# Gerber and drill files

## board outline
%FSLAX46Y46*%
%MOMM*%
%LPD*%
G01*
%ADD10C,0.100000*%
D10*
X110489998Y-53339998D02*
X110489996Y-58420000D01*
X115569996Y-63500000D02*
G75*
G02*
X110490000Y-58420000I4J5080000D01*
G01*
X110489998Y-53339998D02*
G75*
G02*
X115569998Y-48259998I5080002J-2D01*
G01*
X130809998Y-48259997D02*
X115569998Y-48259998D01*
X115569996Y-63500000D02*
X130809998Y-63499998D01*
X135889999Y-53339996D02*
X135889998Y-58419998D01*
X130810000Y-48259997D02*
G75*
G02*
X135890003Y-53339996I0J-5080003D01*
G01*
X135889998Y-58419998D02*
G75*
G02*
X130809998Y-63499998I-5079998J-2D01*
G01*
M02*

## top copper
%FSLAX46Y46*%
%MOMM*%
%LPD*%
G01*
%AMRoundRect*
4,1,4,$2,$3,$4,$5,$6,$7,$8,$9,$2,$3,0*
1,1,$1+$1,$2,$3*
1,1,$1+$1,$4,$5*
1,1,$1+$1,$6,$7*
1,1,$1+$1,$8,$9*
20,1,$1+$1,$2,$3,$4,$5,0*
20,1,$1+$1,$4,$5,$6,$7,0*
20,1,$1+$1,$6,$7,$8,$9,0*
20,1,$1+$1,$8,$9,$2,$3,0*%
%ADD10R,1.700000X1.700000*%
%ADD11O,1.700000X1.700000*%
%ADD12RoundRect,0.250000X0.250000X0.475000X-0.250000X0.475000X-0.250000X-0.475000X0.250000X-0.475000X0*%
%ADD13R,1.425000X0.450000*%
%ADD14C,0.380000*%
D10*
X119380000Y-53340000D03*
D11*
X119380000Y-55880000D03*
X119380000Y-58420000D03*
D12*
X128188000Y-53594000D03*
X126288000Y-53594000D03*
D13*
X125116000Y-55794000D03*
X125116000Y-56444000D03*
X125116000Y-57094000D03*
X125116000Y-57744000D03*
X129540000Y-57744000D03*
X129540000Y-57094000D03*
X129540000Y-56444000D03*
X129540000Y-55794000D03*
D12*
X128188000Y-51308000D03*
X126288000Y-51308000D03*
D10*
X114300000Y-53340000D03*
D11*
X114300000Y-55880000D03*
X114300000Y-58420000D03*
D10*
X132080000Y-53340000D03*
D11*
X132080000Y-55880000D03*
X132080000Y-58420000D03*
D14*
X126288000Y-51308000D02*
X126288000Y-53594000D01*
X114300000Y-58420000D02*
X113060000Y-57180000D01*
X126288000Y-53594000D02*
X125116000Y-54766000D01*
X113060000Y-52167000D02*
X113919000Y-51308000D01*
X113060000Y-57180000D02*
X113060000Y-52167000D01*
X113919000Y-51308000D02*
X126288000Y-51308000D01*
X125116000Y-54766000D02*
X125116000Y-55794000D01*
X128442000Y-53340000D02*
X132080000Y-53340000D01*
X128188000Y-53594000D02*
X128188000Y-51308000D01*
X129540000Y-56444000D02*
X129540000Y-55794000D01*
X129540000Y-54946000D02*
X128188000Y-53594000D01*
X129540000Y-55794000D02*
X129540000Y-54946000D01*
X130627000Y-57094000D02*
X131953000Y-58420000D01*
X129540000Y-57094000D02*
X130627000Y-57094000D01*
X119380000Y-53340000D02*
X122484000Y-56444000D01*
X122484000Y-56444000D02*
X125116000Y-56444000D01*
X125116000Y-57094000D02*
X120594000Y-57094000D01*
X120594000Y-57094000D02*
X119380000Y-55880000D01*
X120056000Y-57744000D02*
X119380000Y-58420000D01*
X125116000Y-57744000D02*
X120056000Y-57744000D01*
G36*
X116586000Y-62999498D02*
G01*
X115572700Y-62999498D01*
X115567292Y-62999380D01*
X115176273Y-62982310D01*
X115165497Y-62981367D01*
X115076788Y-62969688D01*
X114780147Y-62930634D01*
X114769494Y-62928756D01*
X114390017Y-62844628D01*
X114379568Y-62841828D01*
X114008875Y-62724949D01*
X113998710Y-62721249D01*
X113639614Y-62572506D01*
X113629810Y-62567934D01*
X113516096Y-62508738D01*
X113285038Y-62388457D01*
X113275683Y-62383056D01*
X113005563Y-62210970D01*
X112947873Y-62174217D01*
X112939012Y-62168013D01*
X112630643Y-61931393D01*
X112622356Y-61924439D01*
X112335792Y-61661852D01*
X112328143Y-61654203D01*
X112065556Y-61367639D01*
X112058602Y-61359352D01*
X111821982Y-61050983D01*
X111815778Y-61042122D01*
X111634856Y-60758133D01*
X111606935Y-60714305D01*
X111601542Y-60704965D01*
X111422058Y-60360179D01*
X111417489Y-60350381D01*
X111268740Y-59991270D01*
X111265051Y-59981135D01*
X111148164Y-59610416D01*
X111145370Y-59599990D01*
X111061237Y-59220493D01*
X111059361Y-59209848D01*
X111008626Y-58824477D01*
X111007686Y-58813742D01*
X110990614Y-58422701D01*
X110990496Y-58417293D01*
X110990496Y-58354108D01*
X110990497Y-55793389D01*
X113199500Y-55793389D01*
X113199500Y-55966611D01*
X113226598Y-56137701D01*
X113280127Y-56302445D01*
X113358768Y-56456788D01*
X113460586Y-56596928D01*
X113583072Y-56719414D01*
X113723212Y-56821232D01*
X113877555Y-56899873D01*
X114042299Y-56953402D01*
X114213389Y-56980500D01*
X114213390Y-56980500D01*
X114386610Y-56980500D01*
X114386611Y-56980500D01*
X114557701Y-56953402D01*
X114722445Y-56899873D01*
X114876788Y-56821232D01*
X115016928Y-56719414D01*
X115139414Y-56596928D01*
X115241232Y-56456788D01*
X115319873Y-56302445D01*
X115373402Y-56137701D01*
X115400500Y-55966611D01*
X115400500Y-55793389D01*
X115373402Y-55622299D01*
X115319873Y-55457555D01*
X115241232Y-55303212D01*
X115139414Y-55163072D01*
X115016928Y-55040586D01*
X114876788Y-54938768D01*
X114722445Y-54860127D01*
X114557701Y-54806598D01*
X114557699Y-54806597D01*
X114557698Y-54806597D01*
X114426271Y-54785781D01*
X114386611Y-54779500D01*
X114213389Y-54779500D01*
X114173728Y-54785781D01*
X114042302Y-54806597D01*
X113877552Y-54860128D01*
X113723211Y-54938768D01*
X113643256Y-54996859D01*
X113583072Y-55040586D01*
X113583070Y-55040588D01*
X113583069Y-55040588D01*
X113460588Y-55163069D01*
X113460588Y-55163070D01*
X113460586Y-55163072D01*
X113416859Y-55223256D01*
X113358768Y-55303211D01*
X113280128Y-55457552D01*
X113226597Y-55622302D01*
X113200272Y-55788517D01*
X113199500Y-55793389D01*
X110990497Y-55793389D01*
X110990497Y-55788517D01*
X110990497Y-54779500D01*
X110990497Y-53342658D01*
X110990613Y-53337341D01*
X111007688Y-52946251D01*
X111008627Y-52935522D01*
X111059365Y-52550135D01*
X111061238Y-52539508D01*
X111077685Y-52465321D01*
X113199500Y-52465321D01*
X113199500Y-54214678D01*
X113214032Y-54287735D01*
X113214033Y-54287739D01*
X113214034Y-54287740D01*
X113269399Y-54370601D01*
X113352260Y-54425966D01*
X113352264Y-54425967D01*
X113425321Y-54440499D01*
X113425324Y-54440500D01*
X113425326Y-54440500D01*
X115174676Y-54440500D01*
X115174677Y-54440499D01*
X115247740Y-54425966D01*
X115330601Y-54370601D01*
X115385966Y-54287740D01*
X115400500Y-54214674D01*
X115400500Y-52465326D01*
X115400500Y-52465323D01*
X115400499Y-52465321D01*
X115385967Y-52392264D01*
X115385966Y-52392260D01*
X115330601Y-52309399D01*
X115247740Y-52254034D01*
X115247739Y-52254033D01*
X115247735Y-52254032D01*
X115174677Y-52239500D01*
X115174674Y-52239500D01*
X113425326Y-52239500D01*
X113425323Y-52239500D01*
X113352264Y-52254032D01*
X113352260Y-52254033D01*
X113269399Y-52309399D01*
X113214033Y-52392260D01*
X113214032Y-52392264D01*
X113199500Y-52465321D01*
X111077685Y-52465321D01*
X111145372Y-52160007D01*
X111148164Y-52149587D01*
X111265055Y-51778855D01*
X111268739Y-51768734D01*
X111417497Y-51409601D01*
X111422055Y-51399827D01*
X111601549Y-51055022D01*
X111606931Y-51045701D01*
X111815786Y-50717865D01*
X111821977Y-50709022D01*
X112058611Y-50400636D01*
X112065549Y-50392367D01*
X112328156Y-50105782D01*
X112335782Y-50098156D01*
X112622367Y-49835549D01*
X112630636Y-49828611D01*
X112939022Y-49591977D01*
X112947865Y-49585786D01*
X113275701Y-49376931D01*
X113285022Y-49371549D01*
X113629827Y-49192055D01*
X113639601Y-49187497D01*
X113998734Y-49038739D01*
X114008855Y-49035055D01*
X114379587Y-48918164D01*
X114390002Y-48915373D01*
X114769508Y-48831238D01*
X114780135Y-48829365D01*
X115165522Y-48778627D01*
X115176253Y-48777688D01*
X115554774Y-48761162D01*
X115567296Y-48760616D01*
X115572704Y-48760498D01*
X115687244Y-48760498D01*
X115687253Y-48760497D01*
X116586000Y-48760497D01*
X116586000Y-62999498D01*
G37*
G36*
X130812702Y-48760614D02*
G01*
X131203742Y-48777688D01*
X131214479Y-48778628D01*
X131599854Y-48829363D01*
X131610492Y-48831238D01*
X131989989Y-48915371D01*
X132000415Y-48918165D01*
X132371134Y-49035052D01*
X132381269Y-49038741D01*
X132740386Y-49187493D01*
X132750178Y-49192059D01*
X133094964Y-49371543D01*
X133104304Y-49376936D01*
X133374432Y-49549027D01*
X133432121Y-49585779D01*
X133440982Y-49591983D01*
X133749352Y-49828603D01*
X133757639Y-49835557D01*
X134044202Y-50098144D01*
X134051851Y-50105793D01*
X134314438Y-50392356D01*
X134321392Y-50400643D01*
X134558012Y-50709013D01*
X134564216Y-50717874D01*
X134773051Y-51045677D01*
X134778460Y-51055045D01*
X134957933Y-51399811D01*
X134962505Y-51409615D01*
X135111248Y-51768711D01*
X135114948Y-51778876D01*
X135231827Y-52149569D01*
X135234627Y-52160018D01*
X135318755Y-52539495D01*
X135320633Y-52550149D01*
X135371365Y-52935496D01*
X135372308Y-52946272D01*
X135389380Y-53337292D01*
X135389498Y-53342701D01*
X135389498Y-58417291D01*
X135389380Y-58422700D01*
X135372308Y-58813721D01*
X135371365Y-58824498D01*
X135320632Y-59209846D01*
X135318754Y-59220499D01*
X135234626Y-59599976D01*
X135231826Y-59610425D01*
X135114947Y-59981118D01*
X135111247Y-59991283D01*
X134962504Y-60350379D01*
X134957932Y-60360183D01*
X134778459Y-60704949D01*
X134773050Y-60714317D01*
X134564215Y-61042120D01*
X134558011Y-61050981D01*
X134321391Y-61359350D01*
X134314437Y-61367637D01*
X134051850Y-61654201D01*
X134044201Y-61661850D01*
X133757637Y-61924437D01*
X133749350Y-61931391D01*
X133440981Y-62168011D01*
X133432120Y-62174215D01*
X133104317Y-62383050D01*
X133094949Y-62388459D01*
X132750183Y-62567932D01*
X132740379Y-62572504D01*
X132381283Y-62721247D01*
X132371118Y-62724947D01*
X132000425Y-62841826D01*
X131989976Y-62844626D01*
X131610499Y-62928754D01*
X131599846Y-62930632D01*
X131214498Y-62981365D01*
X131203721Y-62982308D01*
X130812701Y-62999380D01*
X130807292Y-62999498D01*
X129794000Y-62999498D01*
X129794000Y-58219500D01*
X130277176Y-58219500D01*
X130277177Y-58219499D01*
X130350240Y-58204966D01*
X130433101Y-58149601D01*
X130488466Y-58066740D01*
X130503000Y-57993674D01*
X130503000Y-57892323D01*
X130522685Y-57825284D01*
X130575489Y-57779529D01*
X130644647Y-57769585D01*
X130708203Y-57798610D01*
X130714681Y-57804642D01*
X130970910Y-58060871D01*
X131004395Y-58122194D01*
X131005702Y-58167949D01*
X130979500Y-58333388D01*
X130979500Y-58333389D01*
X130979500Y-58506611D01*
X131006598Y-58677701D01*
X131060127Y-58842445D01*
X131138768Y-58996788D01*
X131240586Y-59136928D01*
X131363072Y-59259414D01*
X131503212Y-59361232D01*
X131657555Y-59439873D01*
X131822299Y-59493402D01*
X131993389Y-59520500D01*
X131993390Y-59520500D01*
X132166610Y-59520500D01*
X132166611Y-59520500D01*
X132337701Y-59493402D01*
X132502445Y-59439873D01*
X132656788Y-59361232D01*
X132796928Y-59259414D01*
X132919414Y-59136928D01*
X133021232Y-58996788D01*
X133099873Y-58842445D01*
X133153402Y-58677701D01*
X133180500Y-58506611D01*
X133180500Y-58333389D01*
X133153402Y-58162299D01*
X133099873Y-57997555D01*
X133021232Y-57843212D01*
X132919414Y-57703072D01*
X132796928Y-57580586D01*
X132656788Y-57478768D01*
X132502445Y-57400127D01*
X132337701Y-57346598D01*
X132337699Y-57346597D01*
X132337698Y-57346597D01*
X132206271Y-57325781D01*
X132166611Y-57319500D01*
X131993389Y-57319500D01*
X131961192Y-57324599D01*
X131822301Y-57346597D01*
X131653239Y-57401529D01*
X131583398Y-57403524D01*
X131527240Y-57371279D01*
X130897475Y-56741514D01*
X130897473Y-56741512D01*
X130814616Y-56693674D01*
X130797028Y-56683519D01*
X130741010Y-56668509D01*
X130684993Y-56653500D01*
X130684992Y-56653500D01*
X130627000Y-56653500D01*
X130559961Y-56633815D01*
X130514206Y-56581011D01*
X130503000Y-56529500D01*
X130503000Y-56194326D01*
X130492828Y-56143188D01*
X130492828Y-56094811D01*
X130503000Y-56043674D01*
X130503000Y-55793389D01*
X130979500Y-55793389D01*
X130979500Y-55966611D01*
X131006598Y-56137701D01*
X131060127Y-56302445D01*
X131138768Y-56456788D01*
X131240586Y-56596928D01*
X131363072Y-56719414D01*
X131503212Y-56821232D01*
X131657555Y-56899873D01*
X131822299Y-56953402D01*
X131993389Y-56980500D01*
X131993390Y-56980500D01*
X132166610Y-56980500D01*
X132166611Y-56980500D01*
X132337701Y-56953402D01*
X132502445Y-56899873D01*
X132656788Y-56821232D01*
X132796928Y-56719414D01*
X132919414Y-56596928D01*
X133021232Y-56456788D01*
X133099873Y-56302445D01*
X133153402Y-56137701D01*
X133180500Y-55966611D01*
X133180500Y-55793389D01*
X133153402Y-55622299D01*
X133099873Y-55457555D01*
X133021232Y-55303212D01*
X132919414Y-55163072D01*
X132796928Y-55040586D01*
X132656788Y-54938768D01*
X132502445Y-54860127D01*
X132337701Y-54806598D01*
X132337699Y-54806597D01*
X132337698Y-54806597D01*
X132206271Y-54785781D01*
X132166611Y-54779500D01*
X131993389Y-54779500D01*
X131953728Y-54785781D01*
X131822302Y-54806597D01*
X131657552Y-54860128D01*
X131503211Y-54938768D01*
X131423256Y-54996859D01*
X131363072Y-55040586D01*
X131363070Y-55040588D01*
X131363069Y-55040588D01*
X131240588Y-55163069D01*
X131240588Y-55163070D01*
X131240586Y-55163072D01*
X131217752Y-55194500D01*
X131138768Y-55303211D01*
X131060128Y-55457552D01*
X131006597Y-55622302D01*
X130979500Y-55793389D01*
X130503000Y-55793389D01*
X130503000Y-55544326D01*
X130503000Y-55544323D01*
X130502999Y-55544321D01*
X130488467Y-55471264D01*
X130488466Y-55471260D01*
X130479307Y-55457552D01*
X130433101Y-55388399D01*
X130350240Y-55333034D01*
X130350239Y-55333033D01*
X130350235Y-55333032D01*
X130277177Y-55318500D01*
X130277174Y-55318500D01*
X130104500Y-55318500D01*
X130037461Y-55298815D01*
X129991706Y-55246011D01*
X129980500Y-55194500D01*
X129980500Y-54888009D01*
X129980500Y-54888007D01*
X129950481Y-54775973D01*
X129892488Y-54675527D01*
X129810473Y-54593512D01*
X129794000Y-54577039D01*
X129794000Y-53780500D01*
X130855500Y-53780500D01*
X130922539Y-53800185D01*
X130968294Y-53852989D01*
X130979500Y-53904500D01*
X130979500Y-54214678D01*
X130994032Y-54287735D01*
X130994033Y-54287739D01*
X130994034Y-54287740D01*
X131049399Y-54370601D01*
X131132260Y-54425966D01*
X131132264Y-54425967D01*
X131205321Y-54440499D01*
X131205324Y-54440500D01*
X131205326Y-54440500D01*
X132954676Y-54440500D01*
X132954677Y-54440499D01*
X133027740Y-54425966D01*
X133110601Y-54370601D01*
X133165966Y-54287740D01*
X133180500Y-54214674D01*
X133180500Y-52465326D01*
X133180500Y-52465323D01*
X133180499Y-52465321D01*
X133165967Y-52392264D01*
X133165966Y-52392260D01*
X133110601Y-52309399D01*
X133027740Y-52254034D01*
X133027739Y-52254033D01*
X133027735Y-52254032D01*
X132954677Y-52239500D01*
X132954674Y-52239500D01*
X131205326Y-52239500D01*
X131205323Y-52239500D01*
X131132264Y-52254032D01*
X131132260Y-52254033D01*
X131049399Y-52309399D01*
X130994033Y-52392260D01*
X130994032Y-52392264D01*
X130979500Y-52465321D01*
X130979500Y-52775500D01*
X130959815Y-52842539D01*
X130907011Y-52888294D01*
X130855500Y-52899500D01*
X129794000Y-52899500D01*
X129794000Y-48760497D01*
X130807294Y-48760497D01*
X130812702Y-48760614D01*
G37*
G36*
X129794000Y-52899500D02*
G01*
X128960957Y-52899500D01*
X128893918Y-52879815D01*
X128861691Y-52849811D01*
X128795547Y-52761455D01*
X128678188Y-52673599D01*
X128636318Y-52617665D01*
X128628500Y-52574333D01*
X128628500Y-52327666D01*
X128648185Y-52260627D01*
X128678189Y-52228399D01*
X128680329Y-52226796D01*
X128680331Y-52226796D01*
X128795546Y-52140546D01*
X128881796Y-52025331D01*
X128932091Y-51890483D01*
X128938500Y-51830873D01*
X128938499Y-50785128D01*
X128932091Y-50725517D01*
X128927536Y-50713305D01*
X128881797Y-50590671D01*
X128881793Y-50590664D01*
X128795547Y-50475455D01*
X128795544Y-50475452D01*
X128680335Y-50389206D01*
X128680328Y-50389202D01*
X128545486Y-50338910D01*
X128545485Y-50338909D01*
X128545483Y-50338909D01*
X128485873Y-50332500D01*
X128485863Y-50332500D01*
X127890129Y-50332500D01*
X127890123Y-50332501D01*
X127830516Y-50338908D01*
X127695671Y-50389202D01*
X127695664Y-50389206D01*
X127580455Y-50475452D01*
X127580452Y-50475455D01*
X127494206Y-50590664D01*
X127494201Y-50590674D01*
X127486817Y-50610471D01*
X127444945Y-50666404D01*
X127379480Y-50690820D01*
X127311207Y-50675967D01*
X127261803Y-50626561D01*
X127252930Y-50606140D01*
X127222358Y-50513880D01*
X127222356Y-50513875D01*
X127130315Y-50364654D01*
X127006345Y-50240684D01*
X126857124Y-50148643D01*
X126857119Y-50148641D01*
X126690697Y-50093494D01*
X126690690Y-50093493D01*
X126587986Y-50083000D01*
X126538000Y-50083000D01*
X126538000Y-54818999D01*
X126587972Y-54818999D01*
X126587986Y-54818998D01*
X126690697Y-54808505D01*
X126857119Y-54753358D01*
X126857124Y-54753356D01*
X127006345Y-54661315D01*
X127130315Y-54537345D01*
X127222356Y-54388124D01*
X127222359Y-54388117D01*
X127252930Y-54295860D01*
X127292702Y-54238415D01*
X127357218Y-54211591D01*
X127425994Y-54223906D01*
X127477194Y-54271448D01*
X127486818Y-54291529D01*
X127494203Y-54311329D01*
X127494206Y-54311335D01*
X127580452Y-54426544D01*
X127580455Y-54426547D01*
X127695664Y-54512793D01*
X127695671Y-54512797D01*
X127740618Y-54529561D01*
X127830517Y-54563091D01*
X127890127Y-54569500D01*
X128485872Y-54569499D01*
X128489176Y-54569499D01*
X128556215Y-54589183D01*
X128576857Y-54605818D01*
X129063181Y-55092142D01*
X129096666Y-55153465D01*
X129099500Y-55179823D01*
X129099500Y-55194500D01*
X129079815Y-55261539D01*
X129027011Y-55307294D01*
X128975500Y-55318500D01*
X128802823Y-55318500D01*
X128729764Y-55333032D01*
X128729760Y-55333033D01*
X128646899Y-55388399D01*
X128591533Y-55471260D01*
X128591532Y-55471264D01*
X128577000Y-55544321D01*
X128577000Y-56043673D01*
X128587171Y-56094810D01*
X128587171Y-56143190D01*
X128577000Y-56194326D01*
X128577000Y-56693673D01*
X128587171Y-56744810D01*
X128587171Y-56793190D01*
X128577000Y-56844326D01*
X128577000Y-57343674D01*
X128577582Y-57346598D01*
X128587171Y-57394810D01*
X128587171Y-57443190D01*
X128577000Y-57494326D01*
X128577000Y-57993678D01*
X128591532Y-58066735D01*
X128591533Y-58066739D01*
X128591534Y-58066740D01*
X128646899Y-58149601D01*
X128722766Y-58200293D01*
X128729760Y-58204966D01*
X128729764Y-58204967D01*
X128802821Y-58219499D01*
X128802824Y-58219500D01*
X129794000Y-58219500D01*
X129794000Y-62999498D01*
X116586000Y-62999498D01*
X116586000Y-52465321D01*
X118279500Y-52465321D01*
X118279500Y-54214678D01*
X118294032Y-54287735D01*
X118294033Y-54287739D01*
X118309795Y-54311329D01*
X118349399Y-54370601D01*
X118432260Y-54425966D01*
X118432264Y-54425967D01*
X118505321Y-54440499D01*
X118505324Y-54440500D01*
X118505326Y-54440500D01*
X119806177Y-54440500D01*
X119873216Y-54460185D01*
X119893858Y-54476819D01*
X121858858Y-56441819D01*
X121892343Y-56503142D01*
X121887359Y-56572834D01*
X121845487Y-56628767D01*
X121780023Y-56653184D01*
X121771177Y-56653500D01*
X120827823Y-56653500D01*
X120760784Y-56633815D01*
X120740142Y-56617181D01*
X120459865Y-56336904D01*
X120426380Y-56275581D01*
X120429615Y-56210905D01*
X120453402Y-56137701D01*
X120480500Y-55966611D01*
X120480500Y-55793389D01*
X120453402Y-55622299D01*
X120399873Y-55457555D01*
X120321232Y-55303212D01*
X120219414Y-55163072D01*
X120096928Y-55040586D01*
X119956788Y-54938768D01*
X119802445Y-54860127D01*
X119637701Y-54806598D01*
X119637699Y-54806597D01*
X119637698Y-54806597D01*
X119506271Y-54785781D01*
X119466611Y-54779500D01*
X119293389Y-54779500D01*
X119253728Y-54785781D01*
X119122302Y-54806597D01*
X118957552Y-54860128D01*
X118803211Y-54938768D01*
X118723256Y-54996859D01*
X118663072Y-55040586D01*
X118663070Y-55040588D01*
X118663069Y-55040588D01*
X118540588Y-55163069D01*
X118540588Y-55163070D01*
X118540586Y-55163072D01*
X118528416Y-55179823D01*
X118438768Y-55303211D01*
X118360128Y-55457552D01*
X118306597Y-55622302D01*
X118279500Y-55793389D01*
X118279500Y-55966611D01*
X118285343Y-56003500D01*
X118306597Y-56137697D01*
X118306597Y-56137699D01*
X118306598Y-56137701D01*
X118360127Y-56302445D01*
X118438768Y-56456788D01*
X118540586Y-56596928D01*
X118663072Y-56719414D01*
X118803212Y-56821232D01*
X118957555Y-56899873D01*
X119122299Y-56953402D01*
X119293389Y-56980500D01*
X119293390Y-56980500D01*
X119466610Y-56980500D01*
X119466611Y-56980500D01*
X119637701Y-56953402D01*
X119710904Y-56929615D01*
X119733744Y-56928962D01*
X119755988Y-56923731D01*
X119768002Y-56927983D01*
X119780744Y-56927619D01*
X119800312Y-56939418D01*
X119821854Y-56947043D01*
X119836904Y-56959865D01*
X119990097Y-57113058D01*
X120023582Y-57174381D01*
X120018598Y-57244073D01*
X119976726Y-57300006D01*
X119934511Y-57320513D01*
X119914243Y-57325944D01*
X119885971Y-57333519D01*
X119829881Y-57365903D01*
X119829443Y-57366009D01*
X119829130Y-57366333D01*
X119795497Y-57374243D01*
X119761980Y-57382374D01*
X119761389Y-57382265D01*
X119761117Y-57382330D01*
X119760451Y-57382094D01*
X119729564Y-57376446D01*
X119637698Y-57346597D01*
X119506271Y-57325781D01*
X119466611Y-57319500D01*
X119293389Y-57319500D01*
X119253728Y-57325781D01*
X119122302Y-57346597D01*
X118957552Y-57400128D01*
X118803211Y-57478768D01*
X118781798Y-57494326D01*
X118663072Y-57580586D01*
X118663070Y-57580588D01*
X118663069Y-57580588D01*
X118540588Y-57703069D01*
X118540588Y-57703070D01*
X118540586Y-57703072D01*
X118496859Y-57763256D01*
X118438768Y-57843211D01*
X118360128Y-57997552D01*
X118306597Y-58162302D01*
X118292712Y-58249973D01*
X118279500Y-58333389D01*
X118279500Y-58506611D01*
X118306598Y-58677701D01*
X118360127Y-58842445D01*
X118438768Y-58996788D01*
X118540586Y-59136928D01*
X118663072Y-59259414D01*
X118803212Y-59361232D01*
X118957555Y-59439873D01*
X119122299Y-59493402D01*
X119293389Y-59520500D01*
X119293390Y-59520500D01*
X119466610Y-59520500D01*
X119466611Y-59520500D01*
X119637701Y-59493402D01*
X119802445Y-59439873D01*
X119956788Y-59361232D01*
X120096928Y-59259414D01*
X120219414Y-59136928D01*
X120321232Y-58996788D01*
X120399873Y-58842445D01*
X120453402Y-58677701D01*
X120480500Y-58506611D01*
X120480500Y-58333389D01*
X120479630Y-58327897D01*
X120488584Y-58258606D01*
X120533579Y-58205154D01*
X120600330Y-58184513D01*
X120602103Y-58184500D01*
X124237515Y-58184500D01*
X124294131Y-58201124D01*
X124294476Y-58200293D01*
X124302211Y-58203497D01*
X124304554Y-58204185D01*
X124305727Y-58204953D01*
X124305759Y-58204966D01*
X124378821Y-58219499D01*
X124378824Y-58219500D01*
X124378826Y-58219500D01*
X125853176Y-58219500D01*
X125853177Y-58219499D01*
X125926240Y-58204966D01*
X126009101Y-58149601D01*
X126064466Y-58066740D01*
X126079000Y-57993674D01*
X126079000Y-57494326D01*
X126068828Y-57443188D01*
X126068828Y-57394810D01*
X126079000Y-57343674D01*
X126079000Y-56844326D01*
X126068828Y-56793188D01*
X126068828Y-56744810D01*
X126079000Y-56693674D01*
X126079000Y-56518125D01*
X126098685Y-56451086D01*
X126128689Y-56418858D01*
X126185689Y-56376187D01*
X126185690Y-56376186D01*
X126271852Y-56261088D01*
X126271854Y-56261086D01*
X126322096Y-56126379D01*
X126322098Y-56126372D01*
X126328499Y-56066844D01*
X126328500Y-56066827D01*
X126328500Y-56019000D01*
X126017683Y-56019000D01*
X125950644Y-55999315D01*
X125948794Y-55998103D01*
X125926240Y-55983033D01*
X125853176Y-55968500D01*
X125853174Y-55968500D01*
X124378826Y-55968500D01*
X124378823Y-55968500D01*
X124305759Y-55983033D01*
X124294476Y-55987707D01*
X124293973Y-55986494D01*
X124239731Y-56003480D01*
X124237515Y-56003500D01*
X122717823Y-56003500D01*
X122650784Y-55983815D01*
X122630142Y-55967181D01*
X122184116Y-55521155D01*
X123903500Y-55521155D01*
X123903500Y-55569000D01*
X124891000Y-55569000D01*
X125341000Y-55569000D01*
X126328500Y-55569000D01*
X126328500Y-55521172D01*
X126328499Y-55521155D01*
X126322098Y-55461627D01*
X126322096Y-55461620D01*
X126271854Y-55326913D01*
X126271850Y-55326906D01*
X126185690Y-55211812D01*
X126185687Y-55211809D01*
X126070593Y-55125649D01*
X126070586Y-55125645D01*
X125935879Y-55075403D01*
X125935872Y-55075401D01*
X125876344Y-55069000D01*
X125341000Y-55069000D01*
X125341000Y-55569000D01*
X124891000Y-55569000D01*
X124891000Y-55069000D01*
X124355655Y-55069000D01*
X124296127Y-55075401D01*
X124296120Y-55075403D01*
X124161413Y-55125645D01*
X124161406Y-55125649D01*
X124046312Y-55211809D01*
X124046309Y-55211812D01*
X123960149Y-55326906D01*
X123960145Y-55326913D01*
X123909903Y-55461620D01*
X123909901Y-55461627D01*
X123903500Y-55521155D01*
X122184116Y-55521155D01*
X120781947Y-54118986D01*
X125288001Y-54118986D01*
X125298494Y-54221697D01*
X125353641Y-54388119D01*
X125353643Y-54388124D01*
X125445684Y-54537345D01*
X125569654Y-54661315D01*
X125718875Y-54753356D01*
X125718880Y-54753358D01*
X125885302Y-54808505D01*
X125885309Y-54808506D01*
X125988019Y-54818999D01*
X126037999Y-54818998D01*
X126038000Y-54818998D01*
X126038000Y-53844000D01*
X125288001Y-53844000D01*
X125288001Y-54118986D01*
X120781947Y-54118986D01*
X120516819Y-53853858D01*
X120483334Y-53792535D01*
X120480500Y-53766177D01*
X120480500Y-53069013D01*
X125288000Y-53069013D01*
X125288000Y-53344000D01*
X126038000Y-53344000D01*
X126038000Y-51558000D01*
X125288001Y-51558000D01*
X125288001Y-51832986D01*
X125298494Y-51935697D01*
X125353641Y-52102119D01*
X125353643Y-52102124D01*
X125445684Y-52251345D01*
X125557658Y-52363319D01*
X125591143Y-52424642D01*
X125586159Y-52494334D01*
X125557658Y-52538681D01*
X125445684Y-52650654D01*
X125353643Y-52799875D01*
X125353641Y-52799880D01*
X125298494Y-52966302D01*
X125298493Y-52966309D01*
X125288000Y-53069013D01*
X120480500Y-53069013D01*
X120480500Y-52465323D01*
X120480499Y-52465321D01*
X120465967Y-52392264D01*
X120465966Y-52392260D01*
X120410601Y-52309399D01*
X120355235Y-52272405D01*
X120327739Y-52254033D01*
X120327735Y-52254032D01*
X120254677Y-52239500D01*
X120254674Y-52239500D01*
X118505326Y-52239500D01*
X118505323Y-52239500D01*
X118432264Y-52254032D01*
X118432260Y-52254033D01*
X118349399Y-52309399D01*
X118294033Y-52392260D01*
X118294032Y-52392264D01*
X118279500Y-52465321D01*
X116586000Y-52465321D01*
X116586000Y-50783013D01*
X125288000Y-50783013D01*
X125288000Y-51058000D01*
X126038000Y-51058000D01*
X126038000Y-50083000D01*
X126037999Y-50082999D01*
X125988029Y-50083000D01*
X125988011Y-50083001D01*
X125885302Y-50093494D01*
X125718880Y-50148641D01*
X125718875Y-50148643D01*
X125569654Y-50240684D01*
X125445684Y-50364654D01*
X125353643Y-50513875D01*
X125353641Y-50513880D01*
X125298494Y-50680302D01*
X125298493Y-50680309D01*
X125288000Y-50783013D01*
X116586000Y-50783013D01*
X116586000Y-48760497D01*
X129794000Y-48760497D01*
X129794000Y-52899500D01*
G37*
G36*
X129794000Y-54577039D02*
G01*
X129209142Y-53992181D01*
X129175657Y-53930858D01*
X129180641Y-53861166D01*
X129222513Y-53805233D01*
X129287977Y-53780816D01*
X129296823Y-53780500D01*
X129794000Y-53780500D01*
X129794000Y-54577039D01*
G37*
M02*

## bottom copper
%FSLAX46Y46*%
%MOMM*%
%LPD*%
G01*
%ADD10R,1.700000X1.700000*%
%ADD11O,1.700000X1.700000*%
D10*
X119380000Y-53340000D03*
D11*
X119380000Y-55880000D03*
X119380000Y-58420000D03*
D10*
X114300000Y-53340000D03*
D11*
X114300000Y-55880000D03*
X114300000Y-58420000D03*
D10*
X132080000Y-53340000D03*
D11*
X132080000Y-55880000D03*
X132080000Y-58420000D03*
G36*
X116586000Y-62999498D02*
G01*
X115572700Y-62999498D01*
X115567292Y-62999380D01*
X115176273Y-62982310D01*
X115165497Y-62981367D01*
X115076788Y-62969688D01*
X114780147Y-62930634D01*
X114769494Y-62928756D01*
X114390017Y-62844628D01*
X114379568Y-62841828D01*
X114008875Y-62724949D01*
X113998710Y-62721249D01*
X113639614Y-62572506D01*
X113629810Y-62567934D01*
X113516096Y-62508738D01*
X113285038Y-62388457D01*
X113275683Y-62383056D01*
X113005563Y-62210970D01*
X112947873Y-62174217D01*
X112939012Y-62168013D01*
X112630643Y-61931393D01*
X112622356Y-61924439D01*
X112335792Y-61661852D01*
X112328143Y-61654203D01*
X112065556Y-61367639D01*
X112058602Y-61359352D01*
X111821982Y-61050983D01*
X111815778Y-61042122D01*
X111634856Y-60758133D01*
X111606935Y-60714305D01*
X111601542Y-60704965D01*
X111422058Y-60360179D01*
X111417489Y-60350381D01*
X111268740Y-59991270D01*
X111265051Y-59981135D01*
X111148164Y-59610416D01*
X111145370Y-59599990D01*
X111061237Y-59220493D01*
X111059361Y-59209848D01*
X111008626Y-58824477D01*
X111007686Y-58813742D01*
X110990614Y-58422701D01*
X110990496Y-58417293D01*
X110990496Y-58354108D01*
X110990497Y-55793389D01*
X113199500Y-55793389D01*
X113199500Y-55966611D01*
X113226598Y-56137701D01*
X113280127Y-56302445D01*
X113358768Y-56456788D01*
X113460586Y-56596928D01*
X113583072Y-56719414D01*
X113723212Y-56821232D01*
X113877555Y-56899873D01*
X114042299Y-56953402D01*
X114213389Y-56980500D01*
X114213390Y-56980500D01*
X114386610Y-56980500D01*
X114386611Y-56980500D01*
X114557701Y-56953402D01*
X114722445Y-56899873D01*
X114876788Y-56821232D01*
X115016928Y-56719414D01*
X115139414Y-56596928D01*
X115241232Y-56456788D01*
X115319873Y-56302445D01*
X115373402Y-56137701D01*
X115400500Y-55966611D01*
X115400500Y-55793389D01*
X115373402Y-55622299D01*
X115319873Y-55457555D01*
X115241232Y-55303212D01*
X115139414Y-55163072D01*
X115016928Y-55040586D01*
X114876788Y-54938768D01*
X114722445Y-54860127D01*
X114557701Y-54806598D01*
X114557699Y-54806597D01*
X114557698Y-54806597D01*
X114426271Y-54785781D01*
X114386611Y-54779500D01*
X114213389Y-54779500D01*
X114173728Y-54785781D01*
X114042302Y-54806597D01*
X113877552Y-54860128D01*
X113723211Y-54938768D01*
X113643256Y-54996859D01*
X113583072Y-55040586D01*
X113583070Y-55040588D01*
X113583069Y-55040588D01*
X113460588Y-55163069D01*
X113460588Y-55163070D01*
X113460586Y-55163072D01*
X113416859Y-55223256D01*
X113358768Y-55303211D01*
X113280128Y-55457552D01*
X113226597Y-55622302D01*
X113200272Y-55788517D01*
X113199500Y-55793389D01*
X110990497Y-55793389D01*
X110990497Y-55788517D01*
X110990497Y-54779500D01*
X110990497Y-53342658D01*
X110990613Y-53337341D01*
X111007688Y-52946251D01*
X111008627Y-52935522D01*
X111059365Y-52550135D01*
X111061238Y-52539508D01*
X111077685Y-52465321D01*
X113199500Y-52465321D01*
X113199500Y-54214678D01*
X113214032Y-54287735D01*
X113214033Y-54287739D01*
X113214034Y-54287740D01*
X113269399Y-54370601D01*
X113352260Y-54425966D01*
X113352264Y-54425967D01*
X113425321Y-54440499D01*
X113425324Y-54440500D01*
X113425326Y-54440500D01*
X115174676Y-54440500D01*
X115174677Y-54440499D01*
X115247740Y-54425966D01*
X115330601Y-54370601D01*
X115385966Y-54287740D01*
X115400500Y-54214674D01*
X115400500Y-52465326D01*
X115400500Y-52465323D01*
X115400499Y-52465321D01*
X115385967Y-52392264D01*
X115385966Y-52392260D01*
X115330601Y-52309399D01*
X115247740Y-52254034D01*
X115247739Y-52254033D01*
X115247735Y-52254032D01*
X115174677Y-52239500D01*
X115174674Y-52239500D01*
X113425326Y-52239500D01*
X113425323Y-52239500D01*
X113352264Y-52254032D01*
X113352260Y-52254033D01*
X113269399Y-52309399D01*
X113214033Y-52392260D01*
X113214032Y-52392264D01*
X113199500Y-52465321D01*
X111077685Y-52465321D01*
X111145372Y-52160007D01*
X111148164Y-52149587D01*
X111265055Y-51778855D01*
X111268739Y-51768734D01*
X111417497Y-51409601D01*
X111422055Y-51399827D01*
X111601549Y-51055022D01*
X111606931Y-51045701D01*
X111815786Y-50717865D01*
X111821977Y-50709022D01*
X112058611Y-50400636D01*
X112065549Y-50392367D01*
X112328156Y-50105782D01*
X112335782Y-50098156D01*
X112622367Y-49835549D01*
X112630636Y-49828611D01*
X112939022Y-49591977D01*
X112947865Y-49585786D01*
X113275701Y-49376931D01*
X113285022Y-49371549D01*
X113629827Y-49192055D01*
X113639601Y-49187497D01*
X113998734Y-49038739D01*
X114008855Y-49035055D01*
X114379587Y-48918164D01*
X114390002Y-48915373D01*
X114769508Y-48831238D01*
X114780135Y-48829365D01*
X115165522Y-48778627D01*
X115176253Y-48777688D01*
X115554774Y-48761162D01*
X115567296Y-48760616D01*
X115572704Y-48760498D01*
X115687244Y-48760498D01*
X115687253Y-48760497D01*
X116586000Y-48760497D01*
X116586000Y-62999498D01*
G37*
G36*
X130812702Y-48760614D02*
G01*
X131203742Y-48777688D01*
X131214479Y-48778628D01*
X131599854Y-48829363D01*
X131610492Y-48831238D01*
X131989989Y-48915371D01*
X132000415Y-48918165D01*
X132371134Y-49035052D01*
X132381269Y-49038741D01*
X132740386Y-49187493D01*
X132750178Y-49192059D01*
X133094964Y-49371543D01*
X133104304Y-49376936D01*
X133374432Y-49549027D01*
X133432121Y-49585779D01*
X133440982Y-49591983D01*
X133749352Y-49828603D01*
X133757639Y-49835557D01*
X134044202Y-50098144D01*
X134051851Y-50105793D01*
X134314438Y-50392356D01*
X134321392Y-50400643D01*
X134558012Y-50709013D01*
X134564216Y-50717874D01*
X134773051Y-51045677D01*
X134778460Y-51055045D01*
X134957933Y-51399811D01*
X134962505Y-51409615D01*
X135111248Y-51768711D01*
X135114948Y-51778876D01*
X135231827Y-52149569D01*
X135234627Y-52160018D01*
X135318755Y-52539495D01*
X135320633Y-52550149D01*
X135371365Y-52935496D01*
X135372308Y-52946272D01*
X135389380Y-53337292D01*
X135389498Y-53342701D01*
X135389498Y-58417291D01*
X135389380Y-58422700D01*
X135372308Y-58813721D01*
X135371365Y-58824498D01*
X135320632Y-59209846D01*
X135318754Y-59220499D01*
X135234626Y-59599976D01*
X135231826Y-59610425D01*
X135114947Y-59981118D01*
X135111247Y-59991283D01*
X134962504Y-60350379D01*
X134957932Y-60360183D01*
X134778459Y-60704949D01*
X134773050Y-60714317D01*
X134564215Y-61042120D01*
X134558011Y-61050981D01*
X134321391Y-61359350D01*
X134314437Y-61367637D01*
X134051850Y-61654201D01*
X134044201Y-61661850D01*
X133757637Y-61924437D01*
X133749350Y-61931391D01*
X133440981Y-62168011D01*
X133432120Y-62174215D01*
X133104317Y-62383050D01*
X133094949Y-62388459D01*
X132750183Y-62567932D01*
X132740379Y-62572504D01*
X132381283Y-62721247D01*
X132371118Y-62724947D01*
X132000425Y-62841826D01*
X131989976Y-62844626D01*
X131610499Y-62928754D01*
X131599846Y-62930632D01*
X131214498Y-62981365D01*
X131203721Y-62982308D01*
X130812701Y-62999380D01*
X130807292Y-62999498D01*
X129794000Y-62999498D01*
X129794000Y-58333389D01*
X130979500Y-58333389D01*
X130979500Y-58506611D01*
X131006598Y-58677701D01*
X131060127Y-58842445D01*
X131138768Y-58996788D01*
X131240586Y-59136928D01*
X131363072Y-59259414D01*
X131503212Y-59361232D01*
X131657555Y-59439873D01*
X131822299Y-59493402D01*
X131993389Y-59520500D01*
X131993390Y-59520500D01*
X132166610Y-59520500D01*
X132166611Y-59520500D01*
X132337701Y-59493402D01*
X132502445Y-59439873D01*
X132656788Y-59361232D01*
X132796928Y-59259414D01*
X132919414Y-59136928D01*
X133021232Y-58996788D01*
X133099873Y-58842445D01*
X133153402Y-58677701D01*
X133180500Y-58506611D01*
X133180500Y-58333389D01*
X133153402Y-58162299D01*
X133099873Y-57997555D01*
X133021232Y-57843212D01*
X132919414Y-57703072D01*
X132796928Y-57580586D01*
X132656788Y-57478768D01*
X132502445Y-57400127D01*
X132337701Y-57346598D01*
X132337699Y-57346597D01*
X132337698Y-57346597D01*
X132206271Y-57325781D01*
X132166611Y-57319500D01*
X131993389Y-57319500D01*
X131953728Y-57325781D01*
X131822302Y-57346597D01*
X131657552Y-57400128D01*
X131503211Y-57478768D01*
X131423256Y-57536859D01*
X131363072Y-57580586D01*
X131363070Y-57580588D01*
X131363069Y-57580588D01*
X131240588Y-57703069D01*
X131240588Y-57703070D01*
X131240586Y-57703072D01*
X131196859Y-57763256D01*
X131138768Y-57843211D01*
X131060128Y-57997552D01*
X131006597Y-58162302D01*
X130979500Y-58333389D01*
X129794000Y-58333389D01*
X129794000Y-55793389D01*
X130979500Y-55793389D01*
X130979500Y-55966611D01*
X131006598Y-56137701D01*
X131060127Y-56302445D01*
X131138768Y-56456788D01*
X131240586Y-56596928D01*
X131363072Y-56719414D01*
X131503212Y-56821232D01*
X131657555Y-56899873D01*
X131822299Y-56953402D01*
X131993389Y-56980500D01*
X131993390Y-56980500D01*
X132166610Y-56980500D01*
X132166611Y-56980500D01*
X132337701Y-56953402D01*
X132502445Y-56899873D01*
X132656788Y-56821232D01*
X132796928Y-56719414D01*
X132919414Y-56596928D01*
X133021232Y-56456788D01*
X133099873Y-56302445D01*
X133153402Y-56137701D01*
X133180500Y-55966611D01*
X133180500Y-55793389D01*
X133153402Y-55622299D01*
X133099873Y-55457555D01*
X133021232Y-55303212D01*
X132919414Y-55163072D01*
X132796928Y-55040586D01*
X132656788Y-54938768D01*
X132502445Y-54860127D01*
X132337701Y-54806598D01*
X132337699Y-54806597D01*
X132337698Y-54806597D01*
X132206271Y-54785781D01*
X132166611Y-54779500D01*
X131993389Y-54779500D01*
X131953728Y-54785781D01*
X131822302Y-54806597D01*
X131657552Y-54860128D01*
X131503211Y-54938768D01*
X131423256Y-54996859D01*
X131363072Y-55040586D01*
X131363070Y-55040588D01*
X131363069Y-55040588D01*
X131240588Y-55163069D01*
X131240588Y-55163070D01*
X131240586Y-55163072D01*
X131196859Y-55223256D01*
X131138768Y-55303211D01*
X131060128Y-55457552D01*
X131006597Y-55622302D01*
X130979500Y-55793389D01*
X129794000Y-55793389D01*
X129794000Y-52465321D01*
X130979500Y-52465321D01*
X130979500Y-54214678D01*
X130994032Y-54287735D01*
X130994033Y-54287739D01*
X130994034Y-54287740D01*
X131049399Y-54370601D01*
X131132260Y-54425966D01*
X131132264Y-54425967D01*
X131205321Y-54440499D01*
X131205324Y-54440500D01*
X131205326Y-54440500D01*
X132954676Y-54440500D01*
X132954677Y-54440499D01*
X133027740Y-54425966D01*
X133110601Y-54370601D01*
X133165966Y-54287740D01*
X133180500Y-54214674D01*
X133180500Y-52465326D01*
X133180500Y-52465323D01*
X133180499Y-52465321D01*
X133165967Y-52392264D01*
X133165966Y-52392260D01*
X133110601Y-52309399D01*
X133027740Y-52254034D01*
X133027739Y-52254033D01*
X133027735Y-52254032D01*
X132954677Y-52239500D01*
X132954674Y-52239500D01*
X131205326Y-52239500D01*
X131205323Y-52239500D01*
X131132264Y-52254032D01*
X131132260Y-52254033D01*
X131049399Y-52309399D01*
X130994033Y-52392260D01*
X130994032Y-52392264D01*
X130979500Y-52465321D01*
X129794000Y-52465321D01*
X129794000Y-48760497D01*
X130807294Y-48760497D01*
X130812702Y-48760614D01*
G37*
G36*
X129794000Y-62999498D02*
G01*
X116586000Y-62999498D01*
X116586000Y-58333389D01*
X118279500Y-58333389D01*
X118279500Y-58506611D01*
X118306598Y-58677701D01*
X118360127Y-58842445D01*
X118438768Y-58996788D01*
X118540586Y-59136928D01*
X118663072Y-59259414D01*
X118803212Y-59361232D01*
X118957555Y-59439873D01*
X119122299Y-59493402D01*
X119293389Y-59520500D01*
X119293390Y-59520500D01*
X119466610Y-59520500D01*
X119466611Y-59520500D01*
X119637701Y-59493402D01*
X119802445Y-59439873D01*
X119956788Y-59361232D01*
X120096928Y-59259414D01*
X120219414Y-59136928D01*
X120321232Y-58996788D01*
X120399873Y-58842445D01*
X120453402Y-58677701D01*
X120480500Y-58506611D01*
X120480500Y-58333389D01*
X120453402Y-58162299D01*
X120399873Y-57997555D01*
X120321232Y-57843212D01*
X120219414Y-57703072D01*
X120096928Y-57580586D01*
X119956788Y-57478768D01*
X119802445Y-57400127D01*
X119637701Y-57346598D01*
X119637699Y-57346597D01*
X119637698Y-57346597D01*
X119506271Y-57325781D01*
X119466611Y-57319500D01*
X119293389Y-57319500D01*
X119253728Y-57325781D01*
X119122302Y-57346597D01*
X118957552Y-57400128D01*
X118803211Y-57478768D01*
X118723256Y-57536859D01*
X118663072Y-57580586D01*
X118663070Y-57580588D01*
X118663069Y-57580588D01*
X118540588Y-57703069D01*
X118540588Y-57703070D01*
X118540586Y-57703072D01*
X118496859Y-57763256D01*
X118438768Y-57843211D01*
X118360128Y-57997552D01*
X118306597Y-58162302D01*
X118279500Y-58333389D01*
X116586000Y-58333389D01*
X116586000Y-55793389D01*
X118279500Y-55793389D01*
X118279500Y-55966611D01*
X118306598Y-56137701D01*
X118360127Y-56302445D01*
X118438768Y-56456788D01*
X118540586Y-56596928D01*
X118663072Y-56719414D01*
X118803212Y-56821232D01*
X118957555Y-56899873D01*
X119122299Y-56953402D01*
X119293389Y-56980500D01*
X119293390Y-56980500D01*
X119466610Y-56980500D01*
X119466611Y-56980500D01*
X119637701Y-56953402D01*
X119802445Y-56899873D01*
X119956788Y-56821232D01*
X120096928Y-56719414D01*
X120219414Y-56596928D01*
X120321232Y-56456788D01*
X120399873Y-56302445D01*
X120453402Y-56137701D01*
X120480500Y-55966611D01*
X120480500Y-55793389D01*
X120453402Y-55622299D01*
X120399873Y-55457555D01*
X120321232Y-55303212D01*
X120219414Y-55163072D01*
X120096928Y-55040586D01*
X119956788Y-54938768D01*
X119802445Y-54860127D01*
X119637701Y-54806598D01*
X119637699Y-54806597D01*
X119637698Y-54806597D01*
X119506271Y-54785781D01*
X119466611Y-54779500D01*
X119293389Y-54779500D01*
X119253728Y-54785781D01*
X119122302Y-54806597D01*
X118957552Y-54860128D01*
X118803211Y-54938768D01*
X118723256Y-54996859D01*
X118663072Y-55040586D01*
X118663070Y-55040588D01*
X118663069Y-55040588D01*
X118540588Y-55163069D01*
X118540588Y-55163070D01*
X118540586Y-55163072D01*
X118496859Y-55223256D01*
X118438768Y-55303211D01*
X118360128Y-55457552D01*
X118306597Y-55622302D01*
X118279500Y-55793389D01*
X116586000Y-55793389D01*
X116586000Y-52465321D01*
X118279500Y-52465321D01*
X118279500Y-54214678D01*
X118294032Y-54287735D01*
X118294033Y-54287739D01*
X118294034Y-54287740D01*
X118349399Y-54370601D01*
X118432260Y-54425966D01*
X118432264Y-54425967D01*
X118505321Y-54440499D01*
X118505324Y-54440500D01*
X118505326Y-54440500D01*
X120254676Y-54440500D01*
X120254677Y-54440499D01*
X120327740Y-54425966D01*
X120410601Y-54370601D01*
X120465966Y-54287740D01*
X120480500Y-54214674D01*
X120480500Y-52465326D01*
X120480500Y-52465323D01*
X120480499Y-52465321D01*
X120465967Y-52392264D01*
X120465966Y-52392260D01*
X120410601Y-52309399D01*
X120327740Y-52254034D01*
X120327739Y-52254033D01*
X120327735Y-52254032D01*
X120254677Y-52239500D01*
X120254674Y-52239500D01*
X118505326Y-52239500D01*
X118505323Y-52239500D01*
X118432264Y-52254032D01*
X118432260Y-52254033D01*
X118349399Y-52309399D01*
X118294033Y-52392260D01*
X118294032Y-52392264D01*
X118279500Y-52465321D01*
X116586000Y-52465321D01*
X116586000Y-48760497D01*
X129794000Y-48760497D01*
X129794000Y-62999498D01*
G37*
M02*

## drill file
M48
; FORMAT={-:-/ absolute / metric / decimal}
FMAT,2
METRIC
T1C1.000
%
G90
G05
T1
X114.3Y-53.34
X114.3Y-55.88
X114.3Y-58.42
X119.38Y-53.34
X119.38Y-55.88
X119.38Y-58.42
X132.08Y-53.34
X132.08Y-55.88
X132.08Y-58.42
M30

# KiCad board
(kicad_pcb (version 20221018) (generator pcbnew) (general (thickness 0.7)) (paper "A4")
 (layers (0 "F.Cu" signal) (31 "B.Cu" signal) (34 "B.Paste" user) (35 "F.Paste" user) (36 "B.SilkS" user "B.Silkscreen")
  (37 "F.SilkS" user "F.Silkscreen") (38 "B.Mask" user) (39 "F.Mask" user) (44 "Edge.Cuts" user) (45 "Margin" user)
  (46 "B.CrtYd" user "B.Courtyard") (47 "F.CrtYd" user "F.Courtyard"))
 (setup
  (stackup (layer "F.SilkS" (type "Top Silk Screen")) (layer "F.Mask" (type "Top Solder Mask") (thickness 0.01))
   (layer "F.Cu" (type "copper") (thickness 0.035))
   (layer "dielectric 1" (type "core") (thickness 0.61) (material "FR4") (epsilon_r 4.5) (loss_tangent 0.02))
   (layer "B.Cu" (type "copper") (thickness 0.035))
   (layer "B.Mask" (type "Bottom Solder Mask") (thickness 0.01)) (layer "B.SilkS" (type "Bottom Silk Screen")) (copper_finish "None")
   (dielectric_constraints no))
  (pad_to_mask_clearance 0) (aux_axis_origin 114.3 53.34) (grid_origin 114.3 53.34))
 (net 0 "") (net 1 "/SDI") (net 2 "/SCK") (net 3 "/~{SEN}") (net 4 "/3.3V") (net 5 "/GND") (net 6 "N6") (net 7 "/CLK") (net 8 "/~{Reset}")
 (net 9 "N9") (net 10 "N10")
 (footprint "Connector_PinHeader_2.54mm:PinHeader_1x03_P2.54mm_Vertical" (layer "F.Cu") (at 119.38 53.34)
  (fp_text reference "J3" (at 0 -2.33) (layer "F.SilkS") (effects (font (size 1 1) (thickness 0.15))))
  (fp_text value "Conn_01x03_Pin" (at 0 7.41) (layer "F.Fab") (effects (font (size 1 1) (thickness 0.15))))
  (pad "1" thru_hole rect (at 0 0) (size 1.7 1.7) (drill 1) (layers "*.Cu" "*.Mask") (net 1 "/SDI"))
  (pad "2" thru_hole oval (at 0 2.54) (size 1.7 1.7) (drill 1) (layers "*.Cu" "*.Mask") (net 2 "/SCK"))
  (pad "3" thru_hole oval (at 0 5.08) (size 1.7 1.7) (drill 1) (layers "*.Cu" "*.Mask") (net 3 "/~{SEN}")))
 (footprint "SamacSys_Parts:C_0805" (layer "F.Cu") (at 127.254 53.594 90)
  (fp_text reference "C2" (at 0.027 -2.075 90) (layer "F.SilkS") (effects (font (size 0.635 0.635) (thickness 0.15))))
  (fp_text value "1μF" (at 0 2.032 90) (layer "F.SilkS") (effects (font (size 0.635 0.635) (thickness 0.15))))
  (pad "1" smd roundrect (at 0 0.934 180) (size 1 1.45) (layers "F.Cu" "F.Paste" "F.Mask") (roundrect_rratio 0.25) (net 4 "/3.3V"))
  (pad "2" smd roundrect (at 0 -0.966 180) (size 1 1.45) (layers "F.Cu" "F.Paste" "F.Mask") (roundrect_rratio 0.25) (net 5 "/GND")))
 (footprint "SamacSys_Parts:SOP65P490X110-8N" (layer "F.Cu") (at 127.328 56.769)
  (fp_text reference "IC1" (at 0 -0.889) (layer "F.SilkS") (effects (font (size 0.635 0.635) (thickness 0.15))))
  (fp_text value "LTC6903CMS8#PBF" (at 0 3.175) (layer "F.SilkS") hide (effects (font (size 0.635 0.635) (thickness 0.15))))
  (pad "1" smd rect (at -2.212 -0.975 90) (size 0.45 1.425) (layers "F.Cu" "F.Paste" "F.Mask") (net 5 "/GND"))
  (pad "2" smd rect (at -2.212 -0.325 90) (size 0.45 1.425) (layers "F.Cu" "F.Paste" "F.Mask") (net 1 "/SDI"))
  (pad "3" smd rect (at -2.212 0.325 90) (size 0.45 1.425) (layers "F.Cu" "F.Paste" "F.Mask") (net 2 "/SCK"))
  (pad "4" smd rect (at -2.212 0.975 90) (size 0.45 1.425) (layers "F.Cu" "F.Paste" "F.Mask") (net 3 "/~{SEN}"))
  (pad "5" smd rect (at 2.212 0.975 90) (size 0.45 1.425) (layers "F.Cu" "F.Paste" "F.Mask") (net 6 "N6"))
  (pad "6" smd rect (at 2.212 0.325 90) (size 0.45 1.425) (layers "F.Cu" "F.Paste" "F.Mask") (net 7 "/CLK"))
  (pad "7" smd rect (at 2.212 -0.325 90) (size 0.45 1.425) (layers "F.Cu" "F.Paste" "F.Mask") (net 4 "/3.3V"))
  (pad "8" smd rect (at 2.212 -0.975 90) (size 0.45 1.425) (layers "F.Cu" "F.Paste" "F.Mask") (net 4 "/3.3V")))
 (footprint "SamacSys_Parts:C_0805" (layer "F.Cu") (at 127.254 51.308 90)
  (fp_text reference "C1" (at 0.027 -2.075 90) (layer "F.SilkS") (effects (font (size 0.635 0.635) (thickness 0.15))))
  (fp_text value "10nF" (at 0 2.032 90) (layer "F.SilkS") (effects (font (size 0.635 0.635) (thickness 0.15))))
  (pad "1" smd roundrect (at 0 0.934 180) (size 1 1.45) (layers "F.Cu" "F.Paste" "F.Mask") (roundrect_rratio 0.25) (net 4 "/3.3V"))
  (pad "2" smd roundrect (at 0 -0.966 180) (size 1 1.45) (layers "F.Cu" "F.Paste" "F.Mask") (roundrect_rratio 0.25) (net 5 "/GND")))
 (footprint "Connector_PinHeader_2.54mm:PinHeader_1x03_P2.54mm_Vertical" (layer "B.Cu") (at 114.3 53.34 180)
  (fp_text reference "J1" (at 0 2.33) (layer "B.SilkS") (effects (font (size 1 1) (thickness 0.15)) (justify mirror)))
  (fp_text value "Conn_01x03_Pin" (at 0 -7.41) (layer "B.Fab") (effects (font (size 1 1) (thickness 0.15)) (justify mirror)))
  (pad "1" thru_hole rect (at 0 0 180) (size 1.7 1.7) (drill 1) (layers "*.Cu" "*.Mask") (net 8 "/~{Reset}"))
  (pad "2" thru_hole oval (at 0 -2.54 180) (size 1.7 1.7) (drill 1) (layers "*.Cu" "*.Mask") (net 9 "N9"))
  (pad "3" thru_hole oval (at 0 -5.08 180) (size 1.7 1.7) (drill 1) (layers "*.Cu" "*.Mask") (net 5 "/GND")))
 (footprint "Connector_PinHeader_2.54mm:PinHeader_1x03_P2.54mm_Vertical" (layer "B.Cu") (at 132.08 53.34 180)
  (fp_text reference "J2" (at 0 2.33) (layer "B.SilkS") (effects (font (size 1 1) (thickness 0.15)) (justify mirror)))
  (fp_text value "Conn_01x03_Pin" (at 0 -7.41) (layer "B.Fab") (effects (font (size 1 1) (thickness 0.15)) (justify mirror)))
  (pad "1" thru_hole rect (at 0 0 180) (size 1.7 1.7) (drill 1) (layers "*.Cu" "*.Mask") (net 4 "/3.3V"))
  (pad "2" thru_hole oval (at 0 -2.54 180) (size 1.7 1.7) (drill 1) (layers "*.Cu" "*.Mask") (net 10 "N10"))
  (pad "3" thru_hole oval (at 0 -5.08 180) (size 1.7 1.7) (drill 1) (layers "*.Cu" "*.Mask") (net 7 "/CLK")))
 (gr_line (start 110.489998 53.339998) (end 110.489996 58.42) (stroke (width 0.1) (type default)) (layer "Edge.Cuts"))
 (gr_arc (start 115.569996 63.5) (mid 111.977894 62.012102) (end 110.489996 58.42) (stroke (width 0.1) (type default)) (layer "Edge.Cuts"))
 (gr_arc (start 110.489998 53.339998) (mid 111.977896 49.747896) (end 115.569998 48.259998) (stroke (width 0.1) (type default))
  (layer "Edge.Cuts"))
 (gr_line (start 130.809998 48.259997) (end 115.569998 48.259998) (stroke (width 0.1) (type default)) (layer "Edge.Cuts"))
 (gr_line (start 115.569996 63.5) (end 130.809998 63.499998) (stroke (width 0.1) (type default)) (layer "Edge.Cuts"))
 (gr_line (start 135.889999 53.339996) (end 135.889998 58.419998) (stroke (width 0.1) (type default)) (layer "Edge.Cuts"))
 (gr_arc (start 130.81 48.259997) (mid 134.402101 49.747895) (end 135.889999 53.339996) (stroke (width 0.1) (type default))
  (layer "Edge.Cuts"))
 (gr_arc (start 135.889998 58.419998) (mid 134.4021 62.0121) (end 130.809998 63.499998) (stroke (width 0.1) (type default))
  (layer "Edge.Cuts"))
 (segment (start 126.288 51.308) (end 126.288 53.594) (width 0.38) (layer "F.Cu") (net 5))
 (segment (start 114.3 58.42) (end 113.06 57.18) (width 0.38) (layer "F.Cu") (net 5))
 (segment (start 126.288 53.594) (end 125.116 54.766) (width 0.38) (layer "F.Cu") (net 5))
 (segment (start 113.06 52.167) (end 113.919 51.308) (width 0.38) (layer "F.Cu") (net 5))
 (segment (start 113.06 57.18) (end 113.06 52.167) (width 0.38) (layer "F.Cu") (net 5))
 (segment (start 113.919 51.308) (end 126.288 51.308) (width 0.38) (layer "F.Cu") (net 5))
 (segment (start 125.116 54.766) (end 125.116 55.794) (width 0.38) (layer "F.Cu") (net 5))
 (segment (start 128.442 53.34) (end 132.08 53.34) (width 0.38) (layer "F.Cu") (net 4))
 (segment (start 128.188 53.594) (end 128.188 51.308) (width 0.38) (layer "F.Cu") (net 4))
 (segment (start 129.54 56.444) (end 129.54 55.794) (width 0.38) (layer "F.Cu") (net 4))
 (segment (start 129.54 54.946) (end 128.188 53.594) (width 0.38) (layer "F.Cu") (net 4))
 (segment (start 129.54 55.794) (end 129.54 54.946) (width 0.38) (layer "F.Cu") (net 4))
 (segment (start 130.627 57.094) (end 131.953 58.42) (width 0.38) (layer "F.Cu") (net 7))
 (segment (start 129.54 57.094) (end 130.627 57.094) (width 0.38) (layer "F.Cu") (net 7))
 (segment (start 119.38 53.34) (end 122.484 56.444) (width 0.38) (layer "F.Cu") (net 1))
 (segment (start 122.484 56.444) (end 125.116 56.444) (width 0.38) (layer "F.Cu") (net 1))
 (segment (start 125.116 57.094) (end 120.594 57.094) (width 0.38) (layer "F.Cu") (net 2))
 (segment (start 120.594 57.094) (end 119.38 55.88) (width 0.38) (layer "F.Cu") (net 2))
 (segment (start 120.056 57.744) (end 119.38 58.42) (width 0.38) (layer "F.Cu") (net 3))
 (segment (start 125.116 57.744) (end 120.056 57.744) (width 0.38) (layer "F.Cu") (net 3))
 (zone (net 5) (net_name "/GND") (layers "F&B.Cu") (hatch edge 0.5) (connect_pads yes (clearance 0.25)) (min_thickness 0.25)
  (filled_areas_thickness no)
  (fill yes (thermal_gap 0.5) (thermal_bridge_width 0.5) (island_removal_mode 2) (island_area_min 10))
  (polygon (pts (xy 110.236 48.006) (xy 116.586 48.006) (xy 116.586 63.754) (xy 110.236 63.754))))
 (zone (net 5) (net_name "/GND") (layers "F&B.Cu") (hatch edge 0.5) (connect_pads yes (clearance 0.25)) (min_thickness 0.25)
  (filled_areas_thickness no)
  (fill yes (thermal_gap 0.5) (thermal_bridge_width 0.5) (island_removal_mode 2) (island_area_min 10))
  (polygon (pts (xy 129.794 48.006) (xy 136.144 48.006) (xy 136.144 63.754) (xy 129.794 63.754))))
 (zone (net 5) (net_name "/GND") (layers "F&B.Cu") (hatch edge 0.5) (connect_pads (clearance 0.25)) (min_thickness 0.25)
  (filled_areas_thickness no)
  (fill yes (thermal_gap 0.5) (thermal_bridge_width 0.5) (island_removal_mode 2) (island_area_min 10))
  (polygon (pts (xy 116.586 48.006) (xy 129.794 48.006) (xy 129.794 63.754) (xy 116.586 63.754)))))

